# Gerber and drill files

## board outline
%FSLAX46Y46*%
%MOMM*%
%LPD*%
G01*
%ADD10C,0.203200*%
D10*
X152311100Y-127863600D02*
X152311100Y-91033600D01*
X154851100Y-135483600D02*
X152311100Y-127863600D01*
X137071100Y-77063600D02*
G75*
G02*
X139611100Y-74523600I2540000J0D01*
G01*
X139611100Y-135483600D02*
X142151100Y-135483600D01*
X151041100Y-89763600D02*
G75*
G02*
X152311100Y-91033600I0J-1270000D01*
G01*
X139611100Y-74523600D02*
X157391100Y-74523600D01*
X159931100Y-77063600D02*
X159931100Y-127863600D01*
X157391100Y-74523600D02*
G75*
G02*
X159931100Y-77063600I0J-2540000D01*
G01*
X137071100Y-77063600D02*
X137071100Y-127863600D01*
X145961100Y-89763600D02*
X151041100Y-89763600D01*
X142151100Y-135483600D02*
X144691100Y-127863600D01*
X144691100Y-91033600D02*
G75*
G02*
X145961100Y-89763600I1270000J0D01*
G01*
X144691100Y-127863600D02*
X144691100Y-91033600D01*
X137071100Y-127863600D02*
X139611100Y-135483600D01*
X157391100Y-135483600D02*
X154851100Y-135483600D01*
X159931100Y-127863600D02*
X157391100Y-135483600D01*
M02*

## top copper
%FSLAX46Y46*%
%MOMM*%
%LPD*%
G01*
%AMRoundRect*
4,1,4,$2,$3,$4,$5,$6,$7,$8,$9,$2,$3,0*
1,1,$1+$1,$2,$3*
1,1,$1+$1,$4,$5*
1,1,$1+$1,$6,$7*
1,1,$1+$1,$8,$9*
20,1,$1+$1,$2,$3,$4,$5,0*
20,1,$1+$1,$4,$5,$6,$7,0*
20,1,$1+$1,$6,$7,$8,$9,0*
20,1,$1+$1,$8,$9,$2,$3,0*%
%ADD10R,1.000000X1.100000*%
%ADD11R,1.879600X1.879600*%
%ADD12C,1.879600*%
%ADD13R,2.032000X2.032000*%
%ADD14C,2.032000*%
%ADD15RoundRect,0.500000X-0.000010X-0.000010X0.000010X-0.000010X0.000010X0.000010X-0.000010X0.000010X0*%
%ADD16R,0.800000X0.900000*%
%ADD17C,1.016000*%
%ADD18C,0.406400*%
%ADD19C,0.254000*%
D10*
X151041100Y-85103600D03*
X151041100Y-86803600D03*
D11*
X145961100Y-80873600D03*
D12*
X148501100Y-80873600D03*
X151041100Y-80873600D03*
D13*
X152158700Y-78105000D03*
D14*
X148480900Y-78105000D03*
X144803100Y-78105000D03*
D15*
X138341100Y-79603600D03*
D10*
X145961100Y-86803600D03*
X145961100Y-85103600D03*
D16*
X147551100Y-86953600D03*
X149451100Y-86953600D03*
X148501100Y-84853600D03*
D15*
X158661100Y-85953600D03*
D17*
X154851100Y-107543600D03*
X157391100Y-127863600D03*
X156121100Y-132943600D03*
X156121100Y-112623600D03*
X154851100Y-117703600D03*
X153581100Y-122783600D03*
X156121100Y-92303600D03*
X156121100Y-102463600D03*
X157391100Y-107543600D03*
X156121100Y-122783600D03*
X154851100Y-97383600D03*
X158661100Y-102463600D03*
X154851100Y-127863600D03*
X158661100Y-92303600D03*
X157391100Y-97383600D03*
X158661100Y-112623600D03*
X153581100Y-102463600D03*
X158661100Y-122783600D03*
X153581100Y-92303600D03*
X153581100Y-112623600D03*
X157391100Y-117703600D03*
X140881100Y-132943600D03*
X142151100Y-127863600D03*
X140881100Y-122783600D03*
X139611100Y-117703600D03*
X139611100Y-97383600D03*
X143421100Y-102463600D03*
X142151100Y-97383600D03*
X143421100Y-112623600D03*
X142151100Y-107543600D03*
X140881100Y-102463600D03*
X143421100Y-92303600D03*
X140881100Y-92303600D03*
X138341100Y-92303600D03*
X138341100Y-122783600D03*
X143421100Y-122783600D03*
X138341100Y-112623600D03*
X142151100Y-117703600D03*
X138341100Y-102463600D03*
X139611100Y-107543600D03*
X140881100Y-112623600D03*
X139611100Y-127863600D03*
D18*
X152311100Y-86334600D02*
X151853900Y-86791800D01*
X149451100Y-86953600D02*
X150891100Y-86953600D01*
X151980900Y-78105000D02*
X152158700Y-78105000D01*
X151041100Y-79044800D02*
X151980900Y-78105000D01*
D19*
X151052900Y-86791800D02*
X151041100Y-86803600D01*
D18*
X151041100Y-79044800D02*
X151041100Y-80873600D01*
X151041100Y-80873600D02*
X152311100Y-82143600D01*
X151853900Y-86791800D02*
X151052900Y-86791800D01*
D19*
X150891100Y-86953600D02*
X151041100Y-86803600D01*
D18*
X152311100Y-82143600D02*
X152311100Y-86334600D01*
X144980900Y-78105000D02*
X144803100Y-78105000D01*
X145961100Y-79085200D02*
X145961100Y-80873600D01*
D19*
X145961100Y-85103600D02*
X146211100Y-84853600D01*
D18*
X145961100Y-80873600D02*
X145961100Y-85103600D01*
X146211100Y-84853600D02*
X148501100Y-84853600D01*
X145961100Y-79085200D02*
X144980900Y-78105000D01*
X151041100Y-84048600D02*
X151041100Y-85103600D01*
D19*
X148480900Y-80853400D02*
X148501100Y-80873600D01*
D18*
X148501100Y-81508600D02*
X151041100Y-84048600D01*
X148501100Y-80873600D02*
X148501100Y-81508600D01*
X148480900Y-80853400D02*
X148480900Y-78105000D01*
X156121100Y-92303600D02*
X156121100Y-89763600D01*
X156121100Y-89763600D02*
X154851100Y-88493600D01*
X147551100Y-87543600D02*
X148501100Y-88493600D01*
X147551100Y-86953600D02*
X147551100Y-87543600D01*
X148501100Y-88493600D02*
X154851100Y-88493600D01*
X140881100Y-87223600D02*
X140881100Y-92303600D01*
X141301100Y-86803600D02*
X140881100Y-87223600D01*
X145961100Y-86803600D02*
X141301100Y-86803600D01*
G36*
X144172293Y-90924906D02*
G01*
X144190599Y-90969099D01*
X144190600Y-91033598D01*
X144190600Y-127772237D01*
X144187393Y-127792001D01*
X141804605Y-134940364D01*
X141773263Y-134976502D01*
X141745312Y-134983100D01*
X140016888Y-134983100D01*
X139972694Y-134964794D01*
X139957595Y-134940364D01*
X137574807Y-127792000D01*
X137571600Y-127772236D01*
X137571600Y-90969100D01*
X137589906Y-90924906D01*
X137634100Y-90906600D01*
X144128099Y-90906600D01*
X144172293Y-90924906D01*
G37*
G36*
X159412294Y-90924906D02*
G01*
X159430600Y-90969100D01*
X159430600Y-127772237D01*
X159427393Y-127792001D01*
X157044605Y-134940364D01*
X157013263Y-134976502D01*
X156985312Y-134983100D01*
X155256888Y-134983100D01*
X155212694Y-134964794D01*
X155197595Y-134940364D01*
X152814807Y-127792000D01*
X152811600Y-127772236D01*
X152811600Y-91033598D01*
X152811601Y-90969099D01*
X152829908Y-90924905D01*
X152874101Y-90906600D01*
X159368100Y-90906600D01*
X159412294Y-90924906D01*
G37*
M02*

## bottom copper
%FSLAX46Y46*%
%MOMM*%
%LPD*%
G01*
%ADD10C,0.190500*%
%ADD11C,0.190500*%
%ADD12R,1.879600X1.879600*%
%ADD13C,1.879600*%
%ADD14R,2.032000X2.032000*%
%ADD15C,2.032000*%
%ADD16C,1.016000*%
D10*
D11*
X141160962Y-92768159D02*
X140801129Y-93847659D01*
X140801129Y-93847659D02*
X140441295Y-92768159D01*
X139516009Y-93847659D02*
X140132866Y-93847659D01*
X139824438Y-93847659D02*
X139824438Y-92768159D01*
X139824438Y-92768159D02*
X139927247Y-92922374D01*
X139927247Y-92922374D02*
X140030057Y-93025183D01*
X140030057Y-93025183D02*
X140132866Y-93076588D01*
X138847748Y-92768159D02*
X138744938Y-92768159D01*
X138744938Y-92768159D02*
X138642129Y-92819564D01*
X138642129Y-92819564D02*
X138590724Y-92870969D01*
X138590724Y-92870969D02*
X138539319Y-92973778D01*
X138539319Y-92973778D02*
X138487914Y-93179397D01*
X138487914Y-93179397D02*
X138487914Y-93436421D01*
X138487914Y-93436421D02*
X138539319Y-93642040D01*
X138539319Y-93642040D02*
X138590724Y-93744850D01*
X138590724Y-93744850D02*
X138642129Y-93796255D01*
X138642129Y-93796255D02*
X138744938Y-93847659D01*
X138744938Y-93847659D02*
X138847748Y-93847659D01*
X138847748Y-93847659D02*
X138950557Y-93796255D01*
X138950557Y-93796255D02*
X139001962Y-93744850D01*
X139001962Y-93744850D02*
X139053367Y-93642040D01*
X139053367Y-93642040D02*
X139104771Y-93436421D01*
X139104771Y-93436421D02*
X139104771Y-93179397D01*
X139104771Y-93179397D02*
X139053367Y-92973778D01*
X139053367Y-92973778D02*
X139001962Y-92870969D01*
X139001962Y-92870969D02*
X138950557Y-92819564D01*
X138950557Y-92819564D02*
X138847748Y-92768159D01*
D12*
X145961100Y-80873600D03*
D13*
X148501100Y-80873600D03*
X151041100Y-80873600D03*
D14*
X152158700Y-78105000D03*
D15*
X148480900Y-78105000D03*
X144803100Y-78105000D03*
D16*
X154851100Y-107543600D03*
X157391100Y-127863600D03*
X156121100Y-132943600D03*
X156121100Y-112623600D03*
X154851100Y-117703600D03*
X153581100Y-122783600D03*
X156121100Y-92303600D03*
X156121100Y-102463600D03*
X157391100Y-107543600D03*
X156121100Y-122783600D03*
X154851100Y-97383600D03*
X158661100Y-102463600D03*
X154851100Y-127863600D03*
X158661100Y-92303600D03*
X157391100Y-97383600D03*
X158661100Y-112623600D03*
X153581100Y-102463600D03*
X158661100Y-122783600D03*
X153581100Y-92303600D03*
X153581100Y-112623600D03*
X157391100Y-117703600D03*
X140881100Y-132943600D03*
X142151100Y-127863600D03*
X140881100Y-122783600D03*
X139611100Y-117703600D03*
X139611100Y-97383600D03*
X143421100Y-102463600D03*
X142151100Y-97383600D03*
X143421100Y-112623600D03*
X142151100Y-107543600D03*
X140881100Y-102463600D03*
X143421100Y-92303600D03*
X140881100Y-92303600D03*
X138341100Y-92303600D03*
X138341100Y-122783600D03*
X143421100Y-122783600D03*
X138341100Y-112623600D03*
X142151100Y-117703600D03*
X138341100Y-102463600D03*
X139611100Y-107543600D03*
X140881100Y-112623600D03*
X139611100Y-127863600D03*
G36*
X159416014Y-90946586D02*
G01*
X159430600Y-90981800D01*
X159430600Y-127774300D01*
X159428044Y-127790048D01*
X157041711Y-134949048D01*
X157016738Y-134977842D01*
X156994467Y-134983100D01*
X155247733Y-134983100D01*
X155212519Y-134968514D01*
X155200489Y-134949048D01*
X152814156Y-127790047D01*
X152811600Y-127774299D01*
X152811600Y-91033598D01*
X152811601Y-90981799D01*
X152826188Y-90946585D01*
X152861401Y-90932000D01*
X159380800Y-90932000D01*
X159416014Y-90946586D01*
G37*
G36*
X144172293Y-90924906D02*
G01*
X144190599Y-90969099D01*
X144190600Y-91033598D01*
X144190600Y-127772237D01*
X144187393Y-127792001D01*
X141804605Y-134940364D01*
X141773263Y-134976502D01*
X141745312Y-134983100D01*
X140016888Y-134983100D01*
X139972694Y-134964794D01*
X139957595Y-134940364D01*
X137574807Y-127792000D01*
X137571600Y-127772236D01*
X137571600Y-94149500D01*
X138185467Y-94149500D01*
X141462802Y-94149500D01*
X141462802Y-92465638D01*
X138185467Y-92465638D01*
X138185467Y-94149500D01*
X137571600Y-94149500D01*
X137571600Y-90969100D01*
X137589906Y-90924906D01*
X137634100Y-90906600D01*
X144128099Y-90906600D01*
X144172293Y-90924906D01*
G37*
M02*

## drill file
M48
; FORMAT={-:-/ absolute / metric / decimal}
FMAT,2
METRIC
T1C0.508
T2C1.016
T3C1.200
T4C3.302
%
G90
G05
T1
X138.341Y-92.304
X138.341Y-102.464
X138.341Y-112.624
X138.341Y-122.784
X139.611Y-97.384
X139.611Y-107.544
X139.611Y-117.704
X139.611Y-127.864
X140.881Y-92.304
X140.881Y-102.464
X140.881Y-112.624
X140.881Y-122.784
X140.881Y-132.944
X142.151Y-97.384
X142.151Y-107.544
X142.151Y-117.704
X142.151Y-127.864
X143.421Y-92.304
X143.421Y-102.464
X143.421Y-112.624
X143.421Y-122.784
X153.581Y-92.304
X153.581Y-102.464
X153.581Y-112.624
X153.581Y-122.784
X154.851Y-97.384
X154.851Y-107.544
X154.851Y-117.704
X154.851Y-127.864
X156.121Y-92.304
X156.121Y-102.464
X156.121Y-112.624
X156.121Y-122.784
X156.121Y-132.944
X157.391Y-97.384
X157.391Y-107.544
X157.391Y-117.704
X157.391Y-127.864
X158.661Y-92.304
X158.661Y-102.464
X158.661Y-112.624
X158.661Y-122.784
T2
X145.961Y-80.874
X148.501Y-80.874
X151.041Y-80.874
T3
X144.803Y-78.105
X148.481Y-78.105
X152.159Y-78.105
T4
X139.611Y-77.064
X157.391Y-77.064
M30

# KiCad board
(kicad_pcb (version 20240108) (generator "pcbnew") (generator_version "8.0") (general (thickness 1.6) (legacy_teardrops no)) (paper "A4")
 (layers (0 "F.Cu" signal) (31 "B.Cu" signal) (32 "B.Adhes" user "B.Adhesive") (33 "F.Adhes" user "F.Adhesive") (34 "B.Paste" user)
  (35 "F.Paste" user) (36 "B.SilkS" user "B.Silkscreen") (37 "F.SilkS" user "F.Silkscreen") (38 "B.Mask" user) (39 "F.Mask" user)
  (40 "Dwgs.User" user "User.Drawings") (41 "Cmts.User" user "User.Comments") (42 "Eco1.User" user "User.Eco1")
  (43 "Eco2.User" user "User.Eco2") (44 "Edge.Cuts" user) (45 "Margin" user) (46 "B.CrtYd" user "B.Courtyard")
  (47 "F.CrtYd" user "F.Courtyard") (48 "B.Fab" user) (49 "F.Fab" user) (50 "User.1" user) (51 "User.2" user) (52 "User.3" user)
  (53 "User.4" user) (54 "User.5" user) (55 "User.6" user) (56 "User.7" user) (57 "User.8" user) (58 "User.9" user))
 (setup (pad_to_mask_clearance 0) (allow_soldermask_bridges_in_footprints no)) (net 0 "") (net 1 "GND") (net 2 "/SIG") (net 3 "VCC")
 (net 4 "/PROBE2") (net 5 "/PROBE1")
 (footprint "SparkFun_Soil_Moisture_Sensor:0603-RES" (layer "F.Cu") (at 151.0411 85.9536 -90)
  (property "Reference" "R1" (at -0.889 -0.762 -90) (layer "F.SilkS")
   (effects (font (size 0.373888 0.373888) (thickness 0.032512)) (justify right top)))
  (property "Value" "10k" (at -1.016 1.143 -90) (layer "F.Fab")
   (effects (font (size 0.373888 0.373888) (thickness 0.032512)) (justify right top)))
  (pad "1" smd rect (at -0.85 0 270) (size 1.1 1) (layers "F.Cu" "F.Paste" "F.Mask") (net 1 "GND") (solder_mask_margin 0.1016)
   (thermal_bridge_angle 0))
  (pad "2" smd rect (at 0.85 0 270) (size 1.1 1) (layers "F.Cu" "F.Paste" "F.Mask") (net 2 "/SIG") (solder_mask_margin 0.1016)
   (thermal_bridge_angle 0)))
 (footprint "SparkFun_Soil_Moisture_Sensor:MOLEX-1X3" (layer "F.Cu") (at 145.9611 80.8736)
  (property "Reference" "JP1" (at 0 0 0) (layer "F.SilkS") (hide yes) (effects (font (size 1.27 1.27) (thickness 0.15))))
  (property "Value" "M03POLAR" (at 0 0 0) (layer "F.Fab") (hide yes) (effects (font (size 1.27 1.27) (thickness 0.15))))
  (pad "1" thru_hole rect (at 0 0) (size 1.8796 1.8796) (drill 1.016) (layers "*.Cu" "*.Mask") (remove_unused_layers no) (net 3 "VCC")
   (solder_mask_margin 0.1016) (thermal_bridge_angle 0))
  (pad "2" thru_hole circle (at 2.54 0) (size 1.8796 1.8796) (drill 1.016) (layers "*.Cu" "*.Mask") (remove_unused_layers no) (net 1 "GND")
   (solder_mask_margin 0.1016) (thermal_bridge_angle 0))
  (pad "3" thru_hole circle (at 5.08 0) (size 1.8796 1.8796) (drill 1.016) (layers "*.Cu" "*.Mask") (remove_unused_layers no) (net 2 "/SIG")
   (solder_mask_margin 0.1016) (thermal_bridge_angle 0)))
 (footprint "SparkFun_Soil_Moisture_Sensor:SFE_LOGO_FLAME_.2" (layer "F.Cu") (at 154.8511 85.9536)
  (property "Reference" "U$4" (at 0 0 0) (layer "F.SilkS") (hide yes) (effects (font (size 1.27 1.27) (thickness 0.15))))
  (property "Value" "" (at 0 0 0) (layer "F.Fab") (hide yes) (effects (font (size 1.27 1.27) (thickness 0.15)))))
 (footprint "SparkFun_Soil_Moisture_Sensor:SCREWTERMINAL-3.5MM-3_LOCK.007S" (layer "F.Cu") (at 151.9809 78.105 180)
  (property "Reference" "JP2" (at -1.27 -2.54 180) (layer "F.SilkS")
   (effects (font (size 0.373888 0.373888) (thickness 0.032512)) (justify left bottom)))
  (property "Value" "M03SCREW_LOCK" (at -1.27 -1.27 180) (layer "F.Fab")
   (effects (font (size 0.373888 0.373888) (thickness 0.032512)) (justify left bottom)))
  (pad "1" thru_hole rect (at -0.1778 0 180) (size 2.032 2.032) (drill 1.2) (layers "*.Cu" "*.Mask") (remove_unused_layers no)
   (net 2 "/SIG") (solder_mask_margin 0.1016) (thermal_bridge_angle 0))
  (pad "2" thru_hole circle (at 3.5 0 180) (size 2.032 2.032) (drill 1.2) (layers "*.Cu" "*.Mask") (remove_unused_layers no) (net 1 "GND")
   (solder_mask_margin 0.1016) (thermal_bridge_angle 0))
  (pad "3" thru_hole circle (at 7.1778 0 180) (size 2.032 2.032) (drill 1.2) (layers "*.Cu" "*.Mask") (remove_unused_layers no)
   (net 3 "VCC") (solder_mask_margin 0.1016) (thermal_bridge_angle 0)))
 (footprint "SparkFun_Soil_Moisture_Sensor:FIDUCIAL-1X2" (layer "F.Cu") (at 138.3411 79.6036)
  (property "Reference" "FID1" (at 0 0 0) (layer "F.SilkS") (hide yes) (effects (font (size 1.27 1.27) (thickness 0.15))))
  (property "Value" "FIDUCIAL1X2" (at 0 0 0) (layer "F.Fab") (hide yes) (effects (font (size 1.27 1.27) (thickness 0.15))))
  (pad "1" smd roundrect (at 0 0) (size 1 1) (layers "F.Cu" "F.Mask") (roundrect_rratio 0.5) (solder_mask_margin 0.1016)
   (thermal_bridge_angle 0)))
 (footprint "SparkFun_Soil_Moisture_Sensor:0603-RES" (layer "F.Cu") (at 145.9611 85.9536 90)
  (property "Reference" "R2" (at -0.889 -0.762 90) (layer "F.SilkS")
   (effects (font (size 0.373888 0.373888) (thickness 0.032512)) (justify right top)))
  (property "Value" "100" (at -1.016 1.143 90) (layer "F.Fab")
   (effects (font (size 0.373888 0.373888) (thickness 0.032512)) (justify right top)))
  (pad "1" smd rect (at -0.85 0 90) (size 1.1 1) (layers "F.Cu" "F.Paste" "F.Mask") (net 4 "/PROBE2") (solder_mask_margin 0.1016)
   (thermal_bridge_angle 0))
  (pad "2" smd rect (at 0.85 0 90) (size 1.1 1) (layers "F.Cu" "F.Paste" "F.Mask") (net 3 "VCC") (solder_mask_margin 0.1016)
   (thermal_bridge_angle 0)))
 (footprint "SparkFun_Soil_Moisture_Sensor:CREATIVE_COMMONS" (layer "F.Cu") (at 129.4511 145.6436)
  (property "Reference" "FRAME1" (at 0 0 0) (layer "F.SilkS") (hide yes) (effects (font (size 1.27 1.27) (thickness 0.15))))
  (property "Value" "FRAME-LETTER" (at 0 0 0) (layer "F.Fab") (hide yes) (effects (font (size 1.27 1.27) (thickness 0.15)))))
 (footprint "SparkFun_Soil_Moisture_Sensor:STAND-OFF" (layer "F.Cu") (at 139.6111 77.0636)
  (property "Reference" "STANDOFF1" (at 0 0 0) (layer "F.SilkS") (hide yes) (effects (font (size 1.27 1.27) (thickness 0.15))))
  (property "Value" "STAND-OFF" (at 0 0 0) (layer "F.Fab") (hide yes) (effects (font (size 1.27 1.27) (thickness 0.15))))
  (pad "" np_thru_hole circle (at 0 0) (size 3.302 3.302) (drill 3.302) (layers "*.Cu" "*.Mask")))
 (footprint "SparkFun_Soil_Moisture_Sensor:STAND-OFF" (layer "F.Cu") (at 157.3911 77.0636)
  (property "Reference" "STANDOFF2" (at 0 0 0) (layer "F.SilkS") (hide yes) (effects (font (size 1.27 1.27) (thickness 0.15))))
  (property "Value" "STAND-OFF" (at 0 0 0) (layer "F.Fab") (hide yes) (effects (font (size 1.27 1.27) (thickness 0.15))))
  (pad "" np_thru_hole circle (at 0 0) (size 3.302 3.302) (drill 3.302) (layers "*.Cu" "*.Mask")))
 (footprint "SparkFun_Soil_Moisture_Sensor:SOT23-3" (layer "F.Cu") (at 148.5011 85.9536)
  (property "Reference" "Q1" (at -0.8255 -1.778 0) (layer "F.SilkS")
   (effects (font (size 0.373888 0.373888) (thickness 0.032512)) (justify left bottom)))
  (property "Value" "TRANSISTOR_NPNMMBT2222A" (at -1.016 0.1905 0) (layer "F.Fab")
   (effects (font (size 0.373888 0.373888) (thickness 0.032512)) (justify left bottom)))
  (pad "1" smd rect (at -0.95 1) (size 0.8 0.9) (layers "F.Cu" "F.Paste" "F.Mask") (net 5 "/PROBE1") (solder_mask_margin 0.1016)
   (thermal_bridge_angle 0))
  (pad "2" smd rect (at 0.95 1) (size 0.8 0.9) (layers "F.Cu" "F.Paste" "F.Mask") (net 2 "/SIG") (solder_mask_margin 0.1016)
   (thermal_bridge_angle 0))
  (pad "3" smd rect (at 0 -1.1) (size 0.8 0.9) (layers "F.Cu" "F.Paste" "F.Mask") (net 3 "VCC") (solder_mask_margin 0.1016)
   (thermal_bridge_angle 0)))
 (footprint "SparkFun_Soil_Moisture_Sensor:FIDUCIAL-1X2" (layer "F.Cu") (at 158.6611 85.9536)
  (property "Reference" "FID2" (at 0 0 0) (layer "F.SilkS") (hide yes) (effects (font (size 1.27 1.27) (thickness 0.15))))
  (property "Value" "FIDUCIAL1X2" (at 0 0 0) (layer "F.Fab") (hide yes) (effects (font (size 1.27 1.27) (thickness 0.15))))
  (pad "1" smd roundrect (at 0 0) (size 1 1) (layers "F.Cu" "F.Mask") (roundrect_rratio 0.5) (solder_mask_margin 0.1016)
   (thermal_bridge_angle 0)))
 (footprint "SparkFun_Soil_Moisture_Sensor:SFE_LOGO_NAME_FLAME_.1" (layer "B.Cu") (at 154.8511 87.2236 180)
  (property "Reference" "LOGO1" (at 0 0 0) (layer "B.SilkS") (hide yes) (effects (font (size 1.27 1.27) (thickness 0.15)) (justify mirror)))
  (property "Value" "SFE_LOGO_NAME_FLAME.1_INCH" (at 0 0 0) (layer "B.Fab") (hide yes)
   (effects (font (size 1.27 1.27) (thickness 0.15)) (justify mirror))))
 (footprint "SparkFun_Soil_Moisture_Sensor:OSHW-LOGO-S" (layer "B.Cu") (at 157.3911 80.8736 180)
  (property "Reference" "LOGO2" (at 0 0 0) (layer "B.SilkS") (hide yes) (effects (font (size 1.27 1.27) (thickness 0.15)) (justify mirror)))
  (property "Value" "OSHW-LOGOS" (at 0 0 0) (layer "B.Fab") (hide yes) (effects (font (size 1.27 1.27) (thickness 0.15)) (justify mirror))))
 (gr_line (start 152.3111 127.8636) (end 152.3111 91.0336) (stroke (width 0.2032) (type solid)) (layer "Edge.Cuts"))
 (gr_line (start 154.8511 135.4836) (end 152.3111 127.8636) (stroke (width 0.2032) (type solid)) (layer "Edge.Cuts"))
 (gr_arc (start 137.0711 77.0636) (mid 137.815049 75.267549) (end 139.6111 74.5236) (stroke (width 0.2032) (type solid)) (layer "Edge.Cuts"))
 (gr_line (start 139.6111 135.4836) (end 142.1511 135.4836) (stroke (width 0.2032) (type solid)) (layer "Edge.Cuts"))
 (gr_arc (start 151.0411 89.7636) (mid 151.939126 90.135574) (end 152.3111 91.0336) (stroke (width 0.2032) (type solid)) (layer "Edge.Cuts"))
 (gr_line (start 139.6111 74.5236) (end 157.3911 74.5236) (stroke (width 0.2032) (type solid)) (layer "Edge.Cuts"))
 (gr_line (start 159.9311 77.0636) (end 159.9311 127.8636) (stroke (width 0.2032) (type solid)) (layer "Edge.Cuts"))
 (gr_arc (start 157.3911 74.5236) (mid 159.187151 75.267549) (end 159.9311 77.0636) (stroke (width 0.2032) (type solid)) (layer "Edge.Cuts"))
 (gr_line (start 137.0711 77.0636) (end 137.0711 127.8636) (stroke (width 0.2032) (type solid)) (layer "Edge.Cuts"))
 (gr_line (start 145.9611 89.7636) (end 151.0411 89.7636) (stroke (width 0.2032) (type solid)) (layer "Edge.Cuts"))
 (gr_line (start 142.1511 135.4836) (end 144.6911 127.8636) (stroke (width 0.2032) (type solid)) (layer "Edge.Cuts"))
 (gr_arc (start 144.6911 91.0336) (mid 145.063074 90.135574) (end 145.9611 89.7636) (stroke (width 0.2032) (type solid)) (layer "Edge.Cuts"))
 (gr_line (start 144.6911 127.8636) (end 144.6911 91.0336) (stroke (width 0.2032) (type solid)) (layer "Edge.Cuts"))
 (gr_line (start 137.0711 127.8636) (end 139.6111 135.4836) (stroke (width 0.2032) (type solid)) (layer "Edge.Cuts"))
 (gr_line (start 157.3911 135.4836) (end 154.8511 135.4836) (stroke (width 0.2032) (type solid)) (layer "Edge.Cuts"))
 (gr_line (start 159.9311 127.8636) (end 157.3911 135.4836) (stroke (width 0.2032) (type solid)) (layer "Edge.Cuts"))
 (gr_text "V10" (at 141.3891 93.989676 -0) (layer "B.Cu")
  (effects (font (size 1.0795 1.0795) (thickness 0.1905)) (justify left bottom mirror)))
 (segment (start 152.3111 86.3346) (end 151.8539 86.7918) (width 0.4064) (layer "F.Cu") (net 2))
 (segment (start 149.4511 86.9536) (end 150.8911 86.9536) (width 0.4064) (layer "F.Cu") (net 2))
 (segment (start 151.9809 78.105) (end 152.1587 78.105) (width 0.4064) (layer "F.Cu") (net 2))
 (segment (start 151.0411 79.0448) (end 151.9809 78.105) (width 0.4064) (layer "F.Cu") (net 2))
 (segment (start 151.0529 86.7918) (end 151.0411 86.8036) (width 0.254) (layer "F.Cu") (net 2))
 (segment (start 151.0411 79.0448) (end 151.0411 80.8736) (width 0.4064) (layer "F.Cu") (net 2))
 (segment (start 151.0411 80.8736) (end 152.3111 82.1436) (width 0.4064) (layer "F.Cu") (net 2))
 (segment (start 151.8539 86.7918) (end 151.0529 86.7918) (width 0.4064) (layer "F.Cu") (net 2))
 (segment (start 150.8911 86.9536) (end 151.0411 86.8036) (width 0.254) (layer "F.Cu") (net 2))
 (segment (start 152.3111 82.1436) (end 152.3111 86.3346) (width 0.4064) (layer "F.Cu") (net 2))
 (segment (start 144.9809 78.105) (end 144.8031 78.105) (width 0.4064) (layer "F.Cu") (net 3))
 (segment (start 145.9611 79.0852) (end 145.9611 80.8736) (width 0.4064) (layer "F.Cu") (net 3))
 (segment (start 145.9611 85.1036) (end 146.2111 84.8536) (width 0.254) (layer "F.Cu") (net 3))
 (segment (start 145.9611 80.8736) (end 145.9611 85.1036) (width 0.4064) (layer "F.Cu") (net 3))
 (segment (start 146.2111 84.8536) (end 148.5011 84.8536) (width 0.4064) (layer "F.Cu") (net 3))
 (segment (start 145.9611 79.0852) (end 144.9809 78.105) (width 0.4064) (layer "F.Cu") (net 3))
 (segment (start 151.0411 84.0486) (end 151.0411 85.1036) (width 0.4064) (layer "F.Cu") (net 1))
 (segment (start 148.4809 80.8534) (end 148.5011 80.8736) (width 0.254) (layer "F.Cu") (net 1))
 (segment (start 148.5011 81.5086) (end 151.0411 84.0486) (width 0.4064) (layer "F.Cu") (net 1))
 (segment (start 148.5011 80.8736) (end 148.5011 81.5086) (width 0.4064) (layer "F.Cu") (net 1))
 (segment (start 148.4809 80.8534) (end 148.4809 78.105) (width 0.4064) (layer "F.Cu") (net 1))
 (segment (start 156.1211 92.3036) (end 156.1211 89.7636) (width 0.4064) (layer "F.Cu") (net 5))
 (segment (start 156.1211 89.7636) (end 154.8511 88.4936) (width 0.4064) (layer "F.Cu") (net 5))
 (segment (start 147.5511 87.5436) (end 148.5011 88.4936) (width 0.4064) (layer "F.Cu") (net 5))
 (segment (start 147.5511 86.9536) (end 147.5511 87.5436) (width 0.4064) (layer "F.Cu") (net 5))
 (segment (start 148.5011 88.4936) (end 154.8511 88.4936) (width 0.4064) (layer "F.Cu") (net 5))
 (via (at 154.8511 107.5436) (size 1.016) (drill 0.508) (layers "F.Cu" "B.Cu") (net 5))
 (via (at 157.3911 127.8636) (size 1.016) (drill 0.508) (layers "F.Cu" "B.Cu") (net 5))
 (via (at 156.1211 132.9436) (size 1.016) (drill 0.508) (layers "F.Cu" "B.Cu") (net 5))
 (via (at 156.1211 112.6236) (size 1.016) (drill 0.508) (layers "F.Cu" "B.Cu") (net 5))
 (via (at 154.8511 117.7036) (size 1.016) (drill 0.508) (layers "F.Cu" "B.Cu") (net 5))
 (via (at 153.5811 122.7836) (size 1.016) (drill 0.508) (layers "F.Cu" "B.Cu") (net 5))
 (via (at 156.1211 92.3036) (size 1.016) (drill 0.508) (layers "F.Cu" "B.Cu") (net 5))
 (via (at 156.1211 102.4636) (size 1.016) (drill 0.508) (layers "F.Cu" "B.Cu") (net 5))
 (via (at 157.3911 107.5436) (size 1.016) (drill 0.508) (layers "F.Cu" "B.Cu") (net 5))
 (via (at 156.1211 122.7836) (size 1.016) (drill 0.508) (layers "F.Cu" "B.Cu") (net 5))
 (via (at 154.8511 97.3836) (size 1.016) (drill 0.508) (layers "F.Cu" "B.Cu") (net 5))
 (via (at 158.6611 102.4636) (size 1.016) (drill 0.508) (layers "F.Cu" "B.Cu") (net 5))
 (via (at 154.8511 127.8636) (size 1.016) (drill 0.508) (layers "F.Cu" "B.Cu") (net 5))
 (via (at 158.6611 92.3036) (size 1.016) (drill 0.508) (layers "F.Cu" "B.Cu") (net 5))
 (via (at 157.3911 97.3836) (size 1.016) (drill 0.508) (layers "F.Cu" "B.Cu") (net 5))
 (via (at 158.6611 112.6236) (size 1.016) (drill 0.508) (layers "F.Cu" "B.Cu") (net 5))
 (via (at 153.5811 102.4636) (size 1.016) (drill 0.508) (layers "F.Cu" "B.Cu") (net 5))
 (via (at 158.6611 122.7836) (size 1.016) (drill 0.508) (layers "F.Cu" "B.Cu") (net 5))
 (via (at 153.5811 92.3036) (size 1.016) (drill 0.508) (layers "F.Cu" "B.Cu") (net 5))
 (via (at 153.5811 112.6236) (size 1.016) (drill 0.508) (layers "F.Cu" "B.Cu") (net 5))
 (via (at 157.3911 117.7036) (size 1.016) (drill 0.508) (layers "F.Cu" "B.Cu") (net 5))
 (segment (start 140.8811 87.2236) (end 140.8811 92.3036) (width 0.4064) (layer "F.Cu") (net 4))
 (segment (start 141.3011 86.8036) (end 140.8811 87.2236) (width 0.4064) (layer "F.Cu") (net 4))
 (segment (start 145.9611 86.8036) (end 141.3011 86.8036) (width 0.4064) (layer "F.Cu") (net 4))
 (via (at 140.8811 132.9436) (size 1.016) (drill 0.508) (layers "F.Cu" "B.Cu") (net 4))
 (via (at 142.1511 127.8636) (size 1.016) (drill 0.508) (layers "F.Cu" "B.Cu") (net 4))
 (via (at 140.8811 122.7836) (size 1.016) (drill 0.508) (layers "F.Cu" "B.Cu") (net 4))
 (via (at 139.6111 117.7036) (size 1.016) (drill 0.508) (layers "F.Cu" "B.Cu") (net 4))
 (via (at 139.6111 97.3836) (size 1.016) (drill 0.508) (layers "F.Cu" "B.Cu") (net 4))
 (via (at 143.4211 102.4636) (size 1.016) (drill 0.508) (layers "F.Cu" "B.Cu") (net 4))
 (via (at 142.1511 97.3836) (size 1.016) (drill 0.508) (layers "F.Cu" "B.Cu") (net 4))
 (via (at 143.4211 112.6236) (size 1.016) (drill 0.508) (layers "F.Cu" "B.Cu") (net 4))
 (via (at 142.1511 107.5436) (size 1.016) (drill 0.508) (layers "F.Cu" "B.Cu") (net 4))
 (via (at 140.8811 102.4636) (size 1.016) (drill 0.508) (layers "F.Cu" "B.Cu") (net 4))
 (via (at 143.4211 92.3036) (size 1.016) (drill 0.508) (layers "F.Cu" "B.Cu") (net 4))
 (via (at 140.8811 92.3036) (size 1.016) (drill 0.508) (layers "F.Cu" "B.Cu") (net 4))
 (via (at 138.3411 92.3036) (size 1.016) (drill 0.508) (layers "F.Cu" "B.Cu") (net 4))
 (via (at 138.3411 122.7836) (size 1.016) (drill 0.508) (layers "F.Cu" "B.Cu") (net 4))
 (via (at 143.4211 122.7836) (size 1.016) (drill 0.508) (layers "F.Cu" "B.Cu") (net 4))
 (via (at 138.3411 112.6236) (size 1.016) (drill 0.508) (layers "F.Cu" "B.Cu") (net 4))
 (via (at 142.1511 117.7036) (size 1.016) (drill 0.508) (layers "F.Cu" "B.Cu") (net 4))
 (via (at 138.3411 102.4636) (size 1.016) (drill 0.508) (layers "F.Cu" "B.Cu") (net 4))
 (via (at 139.6111 107.5436) (size 1.016) (drill 0.508) (layers "F.Cu" "B.Cu") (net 4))
 (via (at 140.8811 112.6236) (size 1.016) (drill 0.508) (layers "F.Cu" "B.Cu") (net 4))
 (via (at 139.6111 127.8636) (size 1.016) (drill 0.508) (layers "F.Cu" "B.Cu") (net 4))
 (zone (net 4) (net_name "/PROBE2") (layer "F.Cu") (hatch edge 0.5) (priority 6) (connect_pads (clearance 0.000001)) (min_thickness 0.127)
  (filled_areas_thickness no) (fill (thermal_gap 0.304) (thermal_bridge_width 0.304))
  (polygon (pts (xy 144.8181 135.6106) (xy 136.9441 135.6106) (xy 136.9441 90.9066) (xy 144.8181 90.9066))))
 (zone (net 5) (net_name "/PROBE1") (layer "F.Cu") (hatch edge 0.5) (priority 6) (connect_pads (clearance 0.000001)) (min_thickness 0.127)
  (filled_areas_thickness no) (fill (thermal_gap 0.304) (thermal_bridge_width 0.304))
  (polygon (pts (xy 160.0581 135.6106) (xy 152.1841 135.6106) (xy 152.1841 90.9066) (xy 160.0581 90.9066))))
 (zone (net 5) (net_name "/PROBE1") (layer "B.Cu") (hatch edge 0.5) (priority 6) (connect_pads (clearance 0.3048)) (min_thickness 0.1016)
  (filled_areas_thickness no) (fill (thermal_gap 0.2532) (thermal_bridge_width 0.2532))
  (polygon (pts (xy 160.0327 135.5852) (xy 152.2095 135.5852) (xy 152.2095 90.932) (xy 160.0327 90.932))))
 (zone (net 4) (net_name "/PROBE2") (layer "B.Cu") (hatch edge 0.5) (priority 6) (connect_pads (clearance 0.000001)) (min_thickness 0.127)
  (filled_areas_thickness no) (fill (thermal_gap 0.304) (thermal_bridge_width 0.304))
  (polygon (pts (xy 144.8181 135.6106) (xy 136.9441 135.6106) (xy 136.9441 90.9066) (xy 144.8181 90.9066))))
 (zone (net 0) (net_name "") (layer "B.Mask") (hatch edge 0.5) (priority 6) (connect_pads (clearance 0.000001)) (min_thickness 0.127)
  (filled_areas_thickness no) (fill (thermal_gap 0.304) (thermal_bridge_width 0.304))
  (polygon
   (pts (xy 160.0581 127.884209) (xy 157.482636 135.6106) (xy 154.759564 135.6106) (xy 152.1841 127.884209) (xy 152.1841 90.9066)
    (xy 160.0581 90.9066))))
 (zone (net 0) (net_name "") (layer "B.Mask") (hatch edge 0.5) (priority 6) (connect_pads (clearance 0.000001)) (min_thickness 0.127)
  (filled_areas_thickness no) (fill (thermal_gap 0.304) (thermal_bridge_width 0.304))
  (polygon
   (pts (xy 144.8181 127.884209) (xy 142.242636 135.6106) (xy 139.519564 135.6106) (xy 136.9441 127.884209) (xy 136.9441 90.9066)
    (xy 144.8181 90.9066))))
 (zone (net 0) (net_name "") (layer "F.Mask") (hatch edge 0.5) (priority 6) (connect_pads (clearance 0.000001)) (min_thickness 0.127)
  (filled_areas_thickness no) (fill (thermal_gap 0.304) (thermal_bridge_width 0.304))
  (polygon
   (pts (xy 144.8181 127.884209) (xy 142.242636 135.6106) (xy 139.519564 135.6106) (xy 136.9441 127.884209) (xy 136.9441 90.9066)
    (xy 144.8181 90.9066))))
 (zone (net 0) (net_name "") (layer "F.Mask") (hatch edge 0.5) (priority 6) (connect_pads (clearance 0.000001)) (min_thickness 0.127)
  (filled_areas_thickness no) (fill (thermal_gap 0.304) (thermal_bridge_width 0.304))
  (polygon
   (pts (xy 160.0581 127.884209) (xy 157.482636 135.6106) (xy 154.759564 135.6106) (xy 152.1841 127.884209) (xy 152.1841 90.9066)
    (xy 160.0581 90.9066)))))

